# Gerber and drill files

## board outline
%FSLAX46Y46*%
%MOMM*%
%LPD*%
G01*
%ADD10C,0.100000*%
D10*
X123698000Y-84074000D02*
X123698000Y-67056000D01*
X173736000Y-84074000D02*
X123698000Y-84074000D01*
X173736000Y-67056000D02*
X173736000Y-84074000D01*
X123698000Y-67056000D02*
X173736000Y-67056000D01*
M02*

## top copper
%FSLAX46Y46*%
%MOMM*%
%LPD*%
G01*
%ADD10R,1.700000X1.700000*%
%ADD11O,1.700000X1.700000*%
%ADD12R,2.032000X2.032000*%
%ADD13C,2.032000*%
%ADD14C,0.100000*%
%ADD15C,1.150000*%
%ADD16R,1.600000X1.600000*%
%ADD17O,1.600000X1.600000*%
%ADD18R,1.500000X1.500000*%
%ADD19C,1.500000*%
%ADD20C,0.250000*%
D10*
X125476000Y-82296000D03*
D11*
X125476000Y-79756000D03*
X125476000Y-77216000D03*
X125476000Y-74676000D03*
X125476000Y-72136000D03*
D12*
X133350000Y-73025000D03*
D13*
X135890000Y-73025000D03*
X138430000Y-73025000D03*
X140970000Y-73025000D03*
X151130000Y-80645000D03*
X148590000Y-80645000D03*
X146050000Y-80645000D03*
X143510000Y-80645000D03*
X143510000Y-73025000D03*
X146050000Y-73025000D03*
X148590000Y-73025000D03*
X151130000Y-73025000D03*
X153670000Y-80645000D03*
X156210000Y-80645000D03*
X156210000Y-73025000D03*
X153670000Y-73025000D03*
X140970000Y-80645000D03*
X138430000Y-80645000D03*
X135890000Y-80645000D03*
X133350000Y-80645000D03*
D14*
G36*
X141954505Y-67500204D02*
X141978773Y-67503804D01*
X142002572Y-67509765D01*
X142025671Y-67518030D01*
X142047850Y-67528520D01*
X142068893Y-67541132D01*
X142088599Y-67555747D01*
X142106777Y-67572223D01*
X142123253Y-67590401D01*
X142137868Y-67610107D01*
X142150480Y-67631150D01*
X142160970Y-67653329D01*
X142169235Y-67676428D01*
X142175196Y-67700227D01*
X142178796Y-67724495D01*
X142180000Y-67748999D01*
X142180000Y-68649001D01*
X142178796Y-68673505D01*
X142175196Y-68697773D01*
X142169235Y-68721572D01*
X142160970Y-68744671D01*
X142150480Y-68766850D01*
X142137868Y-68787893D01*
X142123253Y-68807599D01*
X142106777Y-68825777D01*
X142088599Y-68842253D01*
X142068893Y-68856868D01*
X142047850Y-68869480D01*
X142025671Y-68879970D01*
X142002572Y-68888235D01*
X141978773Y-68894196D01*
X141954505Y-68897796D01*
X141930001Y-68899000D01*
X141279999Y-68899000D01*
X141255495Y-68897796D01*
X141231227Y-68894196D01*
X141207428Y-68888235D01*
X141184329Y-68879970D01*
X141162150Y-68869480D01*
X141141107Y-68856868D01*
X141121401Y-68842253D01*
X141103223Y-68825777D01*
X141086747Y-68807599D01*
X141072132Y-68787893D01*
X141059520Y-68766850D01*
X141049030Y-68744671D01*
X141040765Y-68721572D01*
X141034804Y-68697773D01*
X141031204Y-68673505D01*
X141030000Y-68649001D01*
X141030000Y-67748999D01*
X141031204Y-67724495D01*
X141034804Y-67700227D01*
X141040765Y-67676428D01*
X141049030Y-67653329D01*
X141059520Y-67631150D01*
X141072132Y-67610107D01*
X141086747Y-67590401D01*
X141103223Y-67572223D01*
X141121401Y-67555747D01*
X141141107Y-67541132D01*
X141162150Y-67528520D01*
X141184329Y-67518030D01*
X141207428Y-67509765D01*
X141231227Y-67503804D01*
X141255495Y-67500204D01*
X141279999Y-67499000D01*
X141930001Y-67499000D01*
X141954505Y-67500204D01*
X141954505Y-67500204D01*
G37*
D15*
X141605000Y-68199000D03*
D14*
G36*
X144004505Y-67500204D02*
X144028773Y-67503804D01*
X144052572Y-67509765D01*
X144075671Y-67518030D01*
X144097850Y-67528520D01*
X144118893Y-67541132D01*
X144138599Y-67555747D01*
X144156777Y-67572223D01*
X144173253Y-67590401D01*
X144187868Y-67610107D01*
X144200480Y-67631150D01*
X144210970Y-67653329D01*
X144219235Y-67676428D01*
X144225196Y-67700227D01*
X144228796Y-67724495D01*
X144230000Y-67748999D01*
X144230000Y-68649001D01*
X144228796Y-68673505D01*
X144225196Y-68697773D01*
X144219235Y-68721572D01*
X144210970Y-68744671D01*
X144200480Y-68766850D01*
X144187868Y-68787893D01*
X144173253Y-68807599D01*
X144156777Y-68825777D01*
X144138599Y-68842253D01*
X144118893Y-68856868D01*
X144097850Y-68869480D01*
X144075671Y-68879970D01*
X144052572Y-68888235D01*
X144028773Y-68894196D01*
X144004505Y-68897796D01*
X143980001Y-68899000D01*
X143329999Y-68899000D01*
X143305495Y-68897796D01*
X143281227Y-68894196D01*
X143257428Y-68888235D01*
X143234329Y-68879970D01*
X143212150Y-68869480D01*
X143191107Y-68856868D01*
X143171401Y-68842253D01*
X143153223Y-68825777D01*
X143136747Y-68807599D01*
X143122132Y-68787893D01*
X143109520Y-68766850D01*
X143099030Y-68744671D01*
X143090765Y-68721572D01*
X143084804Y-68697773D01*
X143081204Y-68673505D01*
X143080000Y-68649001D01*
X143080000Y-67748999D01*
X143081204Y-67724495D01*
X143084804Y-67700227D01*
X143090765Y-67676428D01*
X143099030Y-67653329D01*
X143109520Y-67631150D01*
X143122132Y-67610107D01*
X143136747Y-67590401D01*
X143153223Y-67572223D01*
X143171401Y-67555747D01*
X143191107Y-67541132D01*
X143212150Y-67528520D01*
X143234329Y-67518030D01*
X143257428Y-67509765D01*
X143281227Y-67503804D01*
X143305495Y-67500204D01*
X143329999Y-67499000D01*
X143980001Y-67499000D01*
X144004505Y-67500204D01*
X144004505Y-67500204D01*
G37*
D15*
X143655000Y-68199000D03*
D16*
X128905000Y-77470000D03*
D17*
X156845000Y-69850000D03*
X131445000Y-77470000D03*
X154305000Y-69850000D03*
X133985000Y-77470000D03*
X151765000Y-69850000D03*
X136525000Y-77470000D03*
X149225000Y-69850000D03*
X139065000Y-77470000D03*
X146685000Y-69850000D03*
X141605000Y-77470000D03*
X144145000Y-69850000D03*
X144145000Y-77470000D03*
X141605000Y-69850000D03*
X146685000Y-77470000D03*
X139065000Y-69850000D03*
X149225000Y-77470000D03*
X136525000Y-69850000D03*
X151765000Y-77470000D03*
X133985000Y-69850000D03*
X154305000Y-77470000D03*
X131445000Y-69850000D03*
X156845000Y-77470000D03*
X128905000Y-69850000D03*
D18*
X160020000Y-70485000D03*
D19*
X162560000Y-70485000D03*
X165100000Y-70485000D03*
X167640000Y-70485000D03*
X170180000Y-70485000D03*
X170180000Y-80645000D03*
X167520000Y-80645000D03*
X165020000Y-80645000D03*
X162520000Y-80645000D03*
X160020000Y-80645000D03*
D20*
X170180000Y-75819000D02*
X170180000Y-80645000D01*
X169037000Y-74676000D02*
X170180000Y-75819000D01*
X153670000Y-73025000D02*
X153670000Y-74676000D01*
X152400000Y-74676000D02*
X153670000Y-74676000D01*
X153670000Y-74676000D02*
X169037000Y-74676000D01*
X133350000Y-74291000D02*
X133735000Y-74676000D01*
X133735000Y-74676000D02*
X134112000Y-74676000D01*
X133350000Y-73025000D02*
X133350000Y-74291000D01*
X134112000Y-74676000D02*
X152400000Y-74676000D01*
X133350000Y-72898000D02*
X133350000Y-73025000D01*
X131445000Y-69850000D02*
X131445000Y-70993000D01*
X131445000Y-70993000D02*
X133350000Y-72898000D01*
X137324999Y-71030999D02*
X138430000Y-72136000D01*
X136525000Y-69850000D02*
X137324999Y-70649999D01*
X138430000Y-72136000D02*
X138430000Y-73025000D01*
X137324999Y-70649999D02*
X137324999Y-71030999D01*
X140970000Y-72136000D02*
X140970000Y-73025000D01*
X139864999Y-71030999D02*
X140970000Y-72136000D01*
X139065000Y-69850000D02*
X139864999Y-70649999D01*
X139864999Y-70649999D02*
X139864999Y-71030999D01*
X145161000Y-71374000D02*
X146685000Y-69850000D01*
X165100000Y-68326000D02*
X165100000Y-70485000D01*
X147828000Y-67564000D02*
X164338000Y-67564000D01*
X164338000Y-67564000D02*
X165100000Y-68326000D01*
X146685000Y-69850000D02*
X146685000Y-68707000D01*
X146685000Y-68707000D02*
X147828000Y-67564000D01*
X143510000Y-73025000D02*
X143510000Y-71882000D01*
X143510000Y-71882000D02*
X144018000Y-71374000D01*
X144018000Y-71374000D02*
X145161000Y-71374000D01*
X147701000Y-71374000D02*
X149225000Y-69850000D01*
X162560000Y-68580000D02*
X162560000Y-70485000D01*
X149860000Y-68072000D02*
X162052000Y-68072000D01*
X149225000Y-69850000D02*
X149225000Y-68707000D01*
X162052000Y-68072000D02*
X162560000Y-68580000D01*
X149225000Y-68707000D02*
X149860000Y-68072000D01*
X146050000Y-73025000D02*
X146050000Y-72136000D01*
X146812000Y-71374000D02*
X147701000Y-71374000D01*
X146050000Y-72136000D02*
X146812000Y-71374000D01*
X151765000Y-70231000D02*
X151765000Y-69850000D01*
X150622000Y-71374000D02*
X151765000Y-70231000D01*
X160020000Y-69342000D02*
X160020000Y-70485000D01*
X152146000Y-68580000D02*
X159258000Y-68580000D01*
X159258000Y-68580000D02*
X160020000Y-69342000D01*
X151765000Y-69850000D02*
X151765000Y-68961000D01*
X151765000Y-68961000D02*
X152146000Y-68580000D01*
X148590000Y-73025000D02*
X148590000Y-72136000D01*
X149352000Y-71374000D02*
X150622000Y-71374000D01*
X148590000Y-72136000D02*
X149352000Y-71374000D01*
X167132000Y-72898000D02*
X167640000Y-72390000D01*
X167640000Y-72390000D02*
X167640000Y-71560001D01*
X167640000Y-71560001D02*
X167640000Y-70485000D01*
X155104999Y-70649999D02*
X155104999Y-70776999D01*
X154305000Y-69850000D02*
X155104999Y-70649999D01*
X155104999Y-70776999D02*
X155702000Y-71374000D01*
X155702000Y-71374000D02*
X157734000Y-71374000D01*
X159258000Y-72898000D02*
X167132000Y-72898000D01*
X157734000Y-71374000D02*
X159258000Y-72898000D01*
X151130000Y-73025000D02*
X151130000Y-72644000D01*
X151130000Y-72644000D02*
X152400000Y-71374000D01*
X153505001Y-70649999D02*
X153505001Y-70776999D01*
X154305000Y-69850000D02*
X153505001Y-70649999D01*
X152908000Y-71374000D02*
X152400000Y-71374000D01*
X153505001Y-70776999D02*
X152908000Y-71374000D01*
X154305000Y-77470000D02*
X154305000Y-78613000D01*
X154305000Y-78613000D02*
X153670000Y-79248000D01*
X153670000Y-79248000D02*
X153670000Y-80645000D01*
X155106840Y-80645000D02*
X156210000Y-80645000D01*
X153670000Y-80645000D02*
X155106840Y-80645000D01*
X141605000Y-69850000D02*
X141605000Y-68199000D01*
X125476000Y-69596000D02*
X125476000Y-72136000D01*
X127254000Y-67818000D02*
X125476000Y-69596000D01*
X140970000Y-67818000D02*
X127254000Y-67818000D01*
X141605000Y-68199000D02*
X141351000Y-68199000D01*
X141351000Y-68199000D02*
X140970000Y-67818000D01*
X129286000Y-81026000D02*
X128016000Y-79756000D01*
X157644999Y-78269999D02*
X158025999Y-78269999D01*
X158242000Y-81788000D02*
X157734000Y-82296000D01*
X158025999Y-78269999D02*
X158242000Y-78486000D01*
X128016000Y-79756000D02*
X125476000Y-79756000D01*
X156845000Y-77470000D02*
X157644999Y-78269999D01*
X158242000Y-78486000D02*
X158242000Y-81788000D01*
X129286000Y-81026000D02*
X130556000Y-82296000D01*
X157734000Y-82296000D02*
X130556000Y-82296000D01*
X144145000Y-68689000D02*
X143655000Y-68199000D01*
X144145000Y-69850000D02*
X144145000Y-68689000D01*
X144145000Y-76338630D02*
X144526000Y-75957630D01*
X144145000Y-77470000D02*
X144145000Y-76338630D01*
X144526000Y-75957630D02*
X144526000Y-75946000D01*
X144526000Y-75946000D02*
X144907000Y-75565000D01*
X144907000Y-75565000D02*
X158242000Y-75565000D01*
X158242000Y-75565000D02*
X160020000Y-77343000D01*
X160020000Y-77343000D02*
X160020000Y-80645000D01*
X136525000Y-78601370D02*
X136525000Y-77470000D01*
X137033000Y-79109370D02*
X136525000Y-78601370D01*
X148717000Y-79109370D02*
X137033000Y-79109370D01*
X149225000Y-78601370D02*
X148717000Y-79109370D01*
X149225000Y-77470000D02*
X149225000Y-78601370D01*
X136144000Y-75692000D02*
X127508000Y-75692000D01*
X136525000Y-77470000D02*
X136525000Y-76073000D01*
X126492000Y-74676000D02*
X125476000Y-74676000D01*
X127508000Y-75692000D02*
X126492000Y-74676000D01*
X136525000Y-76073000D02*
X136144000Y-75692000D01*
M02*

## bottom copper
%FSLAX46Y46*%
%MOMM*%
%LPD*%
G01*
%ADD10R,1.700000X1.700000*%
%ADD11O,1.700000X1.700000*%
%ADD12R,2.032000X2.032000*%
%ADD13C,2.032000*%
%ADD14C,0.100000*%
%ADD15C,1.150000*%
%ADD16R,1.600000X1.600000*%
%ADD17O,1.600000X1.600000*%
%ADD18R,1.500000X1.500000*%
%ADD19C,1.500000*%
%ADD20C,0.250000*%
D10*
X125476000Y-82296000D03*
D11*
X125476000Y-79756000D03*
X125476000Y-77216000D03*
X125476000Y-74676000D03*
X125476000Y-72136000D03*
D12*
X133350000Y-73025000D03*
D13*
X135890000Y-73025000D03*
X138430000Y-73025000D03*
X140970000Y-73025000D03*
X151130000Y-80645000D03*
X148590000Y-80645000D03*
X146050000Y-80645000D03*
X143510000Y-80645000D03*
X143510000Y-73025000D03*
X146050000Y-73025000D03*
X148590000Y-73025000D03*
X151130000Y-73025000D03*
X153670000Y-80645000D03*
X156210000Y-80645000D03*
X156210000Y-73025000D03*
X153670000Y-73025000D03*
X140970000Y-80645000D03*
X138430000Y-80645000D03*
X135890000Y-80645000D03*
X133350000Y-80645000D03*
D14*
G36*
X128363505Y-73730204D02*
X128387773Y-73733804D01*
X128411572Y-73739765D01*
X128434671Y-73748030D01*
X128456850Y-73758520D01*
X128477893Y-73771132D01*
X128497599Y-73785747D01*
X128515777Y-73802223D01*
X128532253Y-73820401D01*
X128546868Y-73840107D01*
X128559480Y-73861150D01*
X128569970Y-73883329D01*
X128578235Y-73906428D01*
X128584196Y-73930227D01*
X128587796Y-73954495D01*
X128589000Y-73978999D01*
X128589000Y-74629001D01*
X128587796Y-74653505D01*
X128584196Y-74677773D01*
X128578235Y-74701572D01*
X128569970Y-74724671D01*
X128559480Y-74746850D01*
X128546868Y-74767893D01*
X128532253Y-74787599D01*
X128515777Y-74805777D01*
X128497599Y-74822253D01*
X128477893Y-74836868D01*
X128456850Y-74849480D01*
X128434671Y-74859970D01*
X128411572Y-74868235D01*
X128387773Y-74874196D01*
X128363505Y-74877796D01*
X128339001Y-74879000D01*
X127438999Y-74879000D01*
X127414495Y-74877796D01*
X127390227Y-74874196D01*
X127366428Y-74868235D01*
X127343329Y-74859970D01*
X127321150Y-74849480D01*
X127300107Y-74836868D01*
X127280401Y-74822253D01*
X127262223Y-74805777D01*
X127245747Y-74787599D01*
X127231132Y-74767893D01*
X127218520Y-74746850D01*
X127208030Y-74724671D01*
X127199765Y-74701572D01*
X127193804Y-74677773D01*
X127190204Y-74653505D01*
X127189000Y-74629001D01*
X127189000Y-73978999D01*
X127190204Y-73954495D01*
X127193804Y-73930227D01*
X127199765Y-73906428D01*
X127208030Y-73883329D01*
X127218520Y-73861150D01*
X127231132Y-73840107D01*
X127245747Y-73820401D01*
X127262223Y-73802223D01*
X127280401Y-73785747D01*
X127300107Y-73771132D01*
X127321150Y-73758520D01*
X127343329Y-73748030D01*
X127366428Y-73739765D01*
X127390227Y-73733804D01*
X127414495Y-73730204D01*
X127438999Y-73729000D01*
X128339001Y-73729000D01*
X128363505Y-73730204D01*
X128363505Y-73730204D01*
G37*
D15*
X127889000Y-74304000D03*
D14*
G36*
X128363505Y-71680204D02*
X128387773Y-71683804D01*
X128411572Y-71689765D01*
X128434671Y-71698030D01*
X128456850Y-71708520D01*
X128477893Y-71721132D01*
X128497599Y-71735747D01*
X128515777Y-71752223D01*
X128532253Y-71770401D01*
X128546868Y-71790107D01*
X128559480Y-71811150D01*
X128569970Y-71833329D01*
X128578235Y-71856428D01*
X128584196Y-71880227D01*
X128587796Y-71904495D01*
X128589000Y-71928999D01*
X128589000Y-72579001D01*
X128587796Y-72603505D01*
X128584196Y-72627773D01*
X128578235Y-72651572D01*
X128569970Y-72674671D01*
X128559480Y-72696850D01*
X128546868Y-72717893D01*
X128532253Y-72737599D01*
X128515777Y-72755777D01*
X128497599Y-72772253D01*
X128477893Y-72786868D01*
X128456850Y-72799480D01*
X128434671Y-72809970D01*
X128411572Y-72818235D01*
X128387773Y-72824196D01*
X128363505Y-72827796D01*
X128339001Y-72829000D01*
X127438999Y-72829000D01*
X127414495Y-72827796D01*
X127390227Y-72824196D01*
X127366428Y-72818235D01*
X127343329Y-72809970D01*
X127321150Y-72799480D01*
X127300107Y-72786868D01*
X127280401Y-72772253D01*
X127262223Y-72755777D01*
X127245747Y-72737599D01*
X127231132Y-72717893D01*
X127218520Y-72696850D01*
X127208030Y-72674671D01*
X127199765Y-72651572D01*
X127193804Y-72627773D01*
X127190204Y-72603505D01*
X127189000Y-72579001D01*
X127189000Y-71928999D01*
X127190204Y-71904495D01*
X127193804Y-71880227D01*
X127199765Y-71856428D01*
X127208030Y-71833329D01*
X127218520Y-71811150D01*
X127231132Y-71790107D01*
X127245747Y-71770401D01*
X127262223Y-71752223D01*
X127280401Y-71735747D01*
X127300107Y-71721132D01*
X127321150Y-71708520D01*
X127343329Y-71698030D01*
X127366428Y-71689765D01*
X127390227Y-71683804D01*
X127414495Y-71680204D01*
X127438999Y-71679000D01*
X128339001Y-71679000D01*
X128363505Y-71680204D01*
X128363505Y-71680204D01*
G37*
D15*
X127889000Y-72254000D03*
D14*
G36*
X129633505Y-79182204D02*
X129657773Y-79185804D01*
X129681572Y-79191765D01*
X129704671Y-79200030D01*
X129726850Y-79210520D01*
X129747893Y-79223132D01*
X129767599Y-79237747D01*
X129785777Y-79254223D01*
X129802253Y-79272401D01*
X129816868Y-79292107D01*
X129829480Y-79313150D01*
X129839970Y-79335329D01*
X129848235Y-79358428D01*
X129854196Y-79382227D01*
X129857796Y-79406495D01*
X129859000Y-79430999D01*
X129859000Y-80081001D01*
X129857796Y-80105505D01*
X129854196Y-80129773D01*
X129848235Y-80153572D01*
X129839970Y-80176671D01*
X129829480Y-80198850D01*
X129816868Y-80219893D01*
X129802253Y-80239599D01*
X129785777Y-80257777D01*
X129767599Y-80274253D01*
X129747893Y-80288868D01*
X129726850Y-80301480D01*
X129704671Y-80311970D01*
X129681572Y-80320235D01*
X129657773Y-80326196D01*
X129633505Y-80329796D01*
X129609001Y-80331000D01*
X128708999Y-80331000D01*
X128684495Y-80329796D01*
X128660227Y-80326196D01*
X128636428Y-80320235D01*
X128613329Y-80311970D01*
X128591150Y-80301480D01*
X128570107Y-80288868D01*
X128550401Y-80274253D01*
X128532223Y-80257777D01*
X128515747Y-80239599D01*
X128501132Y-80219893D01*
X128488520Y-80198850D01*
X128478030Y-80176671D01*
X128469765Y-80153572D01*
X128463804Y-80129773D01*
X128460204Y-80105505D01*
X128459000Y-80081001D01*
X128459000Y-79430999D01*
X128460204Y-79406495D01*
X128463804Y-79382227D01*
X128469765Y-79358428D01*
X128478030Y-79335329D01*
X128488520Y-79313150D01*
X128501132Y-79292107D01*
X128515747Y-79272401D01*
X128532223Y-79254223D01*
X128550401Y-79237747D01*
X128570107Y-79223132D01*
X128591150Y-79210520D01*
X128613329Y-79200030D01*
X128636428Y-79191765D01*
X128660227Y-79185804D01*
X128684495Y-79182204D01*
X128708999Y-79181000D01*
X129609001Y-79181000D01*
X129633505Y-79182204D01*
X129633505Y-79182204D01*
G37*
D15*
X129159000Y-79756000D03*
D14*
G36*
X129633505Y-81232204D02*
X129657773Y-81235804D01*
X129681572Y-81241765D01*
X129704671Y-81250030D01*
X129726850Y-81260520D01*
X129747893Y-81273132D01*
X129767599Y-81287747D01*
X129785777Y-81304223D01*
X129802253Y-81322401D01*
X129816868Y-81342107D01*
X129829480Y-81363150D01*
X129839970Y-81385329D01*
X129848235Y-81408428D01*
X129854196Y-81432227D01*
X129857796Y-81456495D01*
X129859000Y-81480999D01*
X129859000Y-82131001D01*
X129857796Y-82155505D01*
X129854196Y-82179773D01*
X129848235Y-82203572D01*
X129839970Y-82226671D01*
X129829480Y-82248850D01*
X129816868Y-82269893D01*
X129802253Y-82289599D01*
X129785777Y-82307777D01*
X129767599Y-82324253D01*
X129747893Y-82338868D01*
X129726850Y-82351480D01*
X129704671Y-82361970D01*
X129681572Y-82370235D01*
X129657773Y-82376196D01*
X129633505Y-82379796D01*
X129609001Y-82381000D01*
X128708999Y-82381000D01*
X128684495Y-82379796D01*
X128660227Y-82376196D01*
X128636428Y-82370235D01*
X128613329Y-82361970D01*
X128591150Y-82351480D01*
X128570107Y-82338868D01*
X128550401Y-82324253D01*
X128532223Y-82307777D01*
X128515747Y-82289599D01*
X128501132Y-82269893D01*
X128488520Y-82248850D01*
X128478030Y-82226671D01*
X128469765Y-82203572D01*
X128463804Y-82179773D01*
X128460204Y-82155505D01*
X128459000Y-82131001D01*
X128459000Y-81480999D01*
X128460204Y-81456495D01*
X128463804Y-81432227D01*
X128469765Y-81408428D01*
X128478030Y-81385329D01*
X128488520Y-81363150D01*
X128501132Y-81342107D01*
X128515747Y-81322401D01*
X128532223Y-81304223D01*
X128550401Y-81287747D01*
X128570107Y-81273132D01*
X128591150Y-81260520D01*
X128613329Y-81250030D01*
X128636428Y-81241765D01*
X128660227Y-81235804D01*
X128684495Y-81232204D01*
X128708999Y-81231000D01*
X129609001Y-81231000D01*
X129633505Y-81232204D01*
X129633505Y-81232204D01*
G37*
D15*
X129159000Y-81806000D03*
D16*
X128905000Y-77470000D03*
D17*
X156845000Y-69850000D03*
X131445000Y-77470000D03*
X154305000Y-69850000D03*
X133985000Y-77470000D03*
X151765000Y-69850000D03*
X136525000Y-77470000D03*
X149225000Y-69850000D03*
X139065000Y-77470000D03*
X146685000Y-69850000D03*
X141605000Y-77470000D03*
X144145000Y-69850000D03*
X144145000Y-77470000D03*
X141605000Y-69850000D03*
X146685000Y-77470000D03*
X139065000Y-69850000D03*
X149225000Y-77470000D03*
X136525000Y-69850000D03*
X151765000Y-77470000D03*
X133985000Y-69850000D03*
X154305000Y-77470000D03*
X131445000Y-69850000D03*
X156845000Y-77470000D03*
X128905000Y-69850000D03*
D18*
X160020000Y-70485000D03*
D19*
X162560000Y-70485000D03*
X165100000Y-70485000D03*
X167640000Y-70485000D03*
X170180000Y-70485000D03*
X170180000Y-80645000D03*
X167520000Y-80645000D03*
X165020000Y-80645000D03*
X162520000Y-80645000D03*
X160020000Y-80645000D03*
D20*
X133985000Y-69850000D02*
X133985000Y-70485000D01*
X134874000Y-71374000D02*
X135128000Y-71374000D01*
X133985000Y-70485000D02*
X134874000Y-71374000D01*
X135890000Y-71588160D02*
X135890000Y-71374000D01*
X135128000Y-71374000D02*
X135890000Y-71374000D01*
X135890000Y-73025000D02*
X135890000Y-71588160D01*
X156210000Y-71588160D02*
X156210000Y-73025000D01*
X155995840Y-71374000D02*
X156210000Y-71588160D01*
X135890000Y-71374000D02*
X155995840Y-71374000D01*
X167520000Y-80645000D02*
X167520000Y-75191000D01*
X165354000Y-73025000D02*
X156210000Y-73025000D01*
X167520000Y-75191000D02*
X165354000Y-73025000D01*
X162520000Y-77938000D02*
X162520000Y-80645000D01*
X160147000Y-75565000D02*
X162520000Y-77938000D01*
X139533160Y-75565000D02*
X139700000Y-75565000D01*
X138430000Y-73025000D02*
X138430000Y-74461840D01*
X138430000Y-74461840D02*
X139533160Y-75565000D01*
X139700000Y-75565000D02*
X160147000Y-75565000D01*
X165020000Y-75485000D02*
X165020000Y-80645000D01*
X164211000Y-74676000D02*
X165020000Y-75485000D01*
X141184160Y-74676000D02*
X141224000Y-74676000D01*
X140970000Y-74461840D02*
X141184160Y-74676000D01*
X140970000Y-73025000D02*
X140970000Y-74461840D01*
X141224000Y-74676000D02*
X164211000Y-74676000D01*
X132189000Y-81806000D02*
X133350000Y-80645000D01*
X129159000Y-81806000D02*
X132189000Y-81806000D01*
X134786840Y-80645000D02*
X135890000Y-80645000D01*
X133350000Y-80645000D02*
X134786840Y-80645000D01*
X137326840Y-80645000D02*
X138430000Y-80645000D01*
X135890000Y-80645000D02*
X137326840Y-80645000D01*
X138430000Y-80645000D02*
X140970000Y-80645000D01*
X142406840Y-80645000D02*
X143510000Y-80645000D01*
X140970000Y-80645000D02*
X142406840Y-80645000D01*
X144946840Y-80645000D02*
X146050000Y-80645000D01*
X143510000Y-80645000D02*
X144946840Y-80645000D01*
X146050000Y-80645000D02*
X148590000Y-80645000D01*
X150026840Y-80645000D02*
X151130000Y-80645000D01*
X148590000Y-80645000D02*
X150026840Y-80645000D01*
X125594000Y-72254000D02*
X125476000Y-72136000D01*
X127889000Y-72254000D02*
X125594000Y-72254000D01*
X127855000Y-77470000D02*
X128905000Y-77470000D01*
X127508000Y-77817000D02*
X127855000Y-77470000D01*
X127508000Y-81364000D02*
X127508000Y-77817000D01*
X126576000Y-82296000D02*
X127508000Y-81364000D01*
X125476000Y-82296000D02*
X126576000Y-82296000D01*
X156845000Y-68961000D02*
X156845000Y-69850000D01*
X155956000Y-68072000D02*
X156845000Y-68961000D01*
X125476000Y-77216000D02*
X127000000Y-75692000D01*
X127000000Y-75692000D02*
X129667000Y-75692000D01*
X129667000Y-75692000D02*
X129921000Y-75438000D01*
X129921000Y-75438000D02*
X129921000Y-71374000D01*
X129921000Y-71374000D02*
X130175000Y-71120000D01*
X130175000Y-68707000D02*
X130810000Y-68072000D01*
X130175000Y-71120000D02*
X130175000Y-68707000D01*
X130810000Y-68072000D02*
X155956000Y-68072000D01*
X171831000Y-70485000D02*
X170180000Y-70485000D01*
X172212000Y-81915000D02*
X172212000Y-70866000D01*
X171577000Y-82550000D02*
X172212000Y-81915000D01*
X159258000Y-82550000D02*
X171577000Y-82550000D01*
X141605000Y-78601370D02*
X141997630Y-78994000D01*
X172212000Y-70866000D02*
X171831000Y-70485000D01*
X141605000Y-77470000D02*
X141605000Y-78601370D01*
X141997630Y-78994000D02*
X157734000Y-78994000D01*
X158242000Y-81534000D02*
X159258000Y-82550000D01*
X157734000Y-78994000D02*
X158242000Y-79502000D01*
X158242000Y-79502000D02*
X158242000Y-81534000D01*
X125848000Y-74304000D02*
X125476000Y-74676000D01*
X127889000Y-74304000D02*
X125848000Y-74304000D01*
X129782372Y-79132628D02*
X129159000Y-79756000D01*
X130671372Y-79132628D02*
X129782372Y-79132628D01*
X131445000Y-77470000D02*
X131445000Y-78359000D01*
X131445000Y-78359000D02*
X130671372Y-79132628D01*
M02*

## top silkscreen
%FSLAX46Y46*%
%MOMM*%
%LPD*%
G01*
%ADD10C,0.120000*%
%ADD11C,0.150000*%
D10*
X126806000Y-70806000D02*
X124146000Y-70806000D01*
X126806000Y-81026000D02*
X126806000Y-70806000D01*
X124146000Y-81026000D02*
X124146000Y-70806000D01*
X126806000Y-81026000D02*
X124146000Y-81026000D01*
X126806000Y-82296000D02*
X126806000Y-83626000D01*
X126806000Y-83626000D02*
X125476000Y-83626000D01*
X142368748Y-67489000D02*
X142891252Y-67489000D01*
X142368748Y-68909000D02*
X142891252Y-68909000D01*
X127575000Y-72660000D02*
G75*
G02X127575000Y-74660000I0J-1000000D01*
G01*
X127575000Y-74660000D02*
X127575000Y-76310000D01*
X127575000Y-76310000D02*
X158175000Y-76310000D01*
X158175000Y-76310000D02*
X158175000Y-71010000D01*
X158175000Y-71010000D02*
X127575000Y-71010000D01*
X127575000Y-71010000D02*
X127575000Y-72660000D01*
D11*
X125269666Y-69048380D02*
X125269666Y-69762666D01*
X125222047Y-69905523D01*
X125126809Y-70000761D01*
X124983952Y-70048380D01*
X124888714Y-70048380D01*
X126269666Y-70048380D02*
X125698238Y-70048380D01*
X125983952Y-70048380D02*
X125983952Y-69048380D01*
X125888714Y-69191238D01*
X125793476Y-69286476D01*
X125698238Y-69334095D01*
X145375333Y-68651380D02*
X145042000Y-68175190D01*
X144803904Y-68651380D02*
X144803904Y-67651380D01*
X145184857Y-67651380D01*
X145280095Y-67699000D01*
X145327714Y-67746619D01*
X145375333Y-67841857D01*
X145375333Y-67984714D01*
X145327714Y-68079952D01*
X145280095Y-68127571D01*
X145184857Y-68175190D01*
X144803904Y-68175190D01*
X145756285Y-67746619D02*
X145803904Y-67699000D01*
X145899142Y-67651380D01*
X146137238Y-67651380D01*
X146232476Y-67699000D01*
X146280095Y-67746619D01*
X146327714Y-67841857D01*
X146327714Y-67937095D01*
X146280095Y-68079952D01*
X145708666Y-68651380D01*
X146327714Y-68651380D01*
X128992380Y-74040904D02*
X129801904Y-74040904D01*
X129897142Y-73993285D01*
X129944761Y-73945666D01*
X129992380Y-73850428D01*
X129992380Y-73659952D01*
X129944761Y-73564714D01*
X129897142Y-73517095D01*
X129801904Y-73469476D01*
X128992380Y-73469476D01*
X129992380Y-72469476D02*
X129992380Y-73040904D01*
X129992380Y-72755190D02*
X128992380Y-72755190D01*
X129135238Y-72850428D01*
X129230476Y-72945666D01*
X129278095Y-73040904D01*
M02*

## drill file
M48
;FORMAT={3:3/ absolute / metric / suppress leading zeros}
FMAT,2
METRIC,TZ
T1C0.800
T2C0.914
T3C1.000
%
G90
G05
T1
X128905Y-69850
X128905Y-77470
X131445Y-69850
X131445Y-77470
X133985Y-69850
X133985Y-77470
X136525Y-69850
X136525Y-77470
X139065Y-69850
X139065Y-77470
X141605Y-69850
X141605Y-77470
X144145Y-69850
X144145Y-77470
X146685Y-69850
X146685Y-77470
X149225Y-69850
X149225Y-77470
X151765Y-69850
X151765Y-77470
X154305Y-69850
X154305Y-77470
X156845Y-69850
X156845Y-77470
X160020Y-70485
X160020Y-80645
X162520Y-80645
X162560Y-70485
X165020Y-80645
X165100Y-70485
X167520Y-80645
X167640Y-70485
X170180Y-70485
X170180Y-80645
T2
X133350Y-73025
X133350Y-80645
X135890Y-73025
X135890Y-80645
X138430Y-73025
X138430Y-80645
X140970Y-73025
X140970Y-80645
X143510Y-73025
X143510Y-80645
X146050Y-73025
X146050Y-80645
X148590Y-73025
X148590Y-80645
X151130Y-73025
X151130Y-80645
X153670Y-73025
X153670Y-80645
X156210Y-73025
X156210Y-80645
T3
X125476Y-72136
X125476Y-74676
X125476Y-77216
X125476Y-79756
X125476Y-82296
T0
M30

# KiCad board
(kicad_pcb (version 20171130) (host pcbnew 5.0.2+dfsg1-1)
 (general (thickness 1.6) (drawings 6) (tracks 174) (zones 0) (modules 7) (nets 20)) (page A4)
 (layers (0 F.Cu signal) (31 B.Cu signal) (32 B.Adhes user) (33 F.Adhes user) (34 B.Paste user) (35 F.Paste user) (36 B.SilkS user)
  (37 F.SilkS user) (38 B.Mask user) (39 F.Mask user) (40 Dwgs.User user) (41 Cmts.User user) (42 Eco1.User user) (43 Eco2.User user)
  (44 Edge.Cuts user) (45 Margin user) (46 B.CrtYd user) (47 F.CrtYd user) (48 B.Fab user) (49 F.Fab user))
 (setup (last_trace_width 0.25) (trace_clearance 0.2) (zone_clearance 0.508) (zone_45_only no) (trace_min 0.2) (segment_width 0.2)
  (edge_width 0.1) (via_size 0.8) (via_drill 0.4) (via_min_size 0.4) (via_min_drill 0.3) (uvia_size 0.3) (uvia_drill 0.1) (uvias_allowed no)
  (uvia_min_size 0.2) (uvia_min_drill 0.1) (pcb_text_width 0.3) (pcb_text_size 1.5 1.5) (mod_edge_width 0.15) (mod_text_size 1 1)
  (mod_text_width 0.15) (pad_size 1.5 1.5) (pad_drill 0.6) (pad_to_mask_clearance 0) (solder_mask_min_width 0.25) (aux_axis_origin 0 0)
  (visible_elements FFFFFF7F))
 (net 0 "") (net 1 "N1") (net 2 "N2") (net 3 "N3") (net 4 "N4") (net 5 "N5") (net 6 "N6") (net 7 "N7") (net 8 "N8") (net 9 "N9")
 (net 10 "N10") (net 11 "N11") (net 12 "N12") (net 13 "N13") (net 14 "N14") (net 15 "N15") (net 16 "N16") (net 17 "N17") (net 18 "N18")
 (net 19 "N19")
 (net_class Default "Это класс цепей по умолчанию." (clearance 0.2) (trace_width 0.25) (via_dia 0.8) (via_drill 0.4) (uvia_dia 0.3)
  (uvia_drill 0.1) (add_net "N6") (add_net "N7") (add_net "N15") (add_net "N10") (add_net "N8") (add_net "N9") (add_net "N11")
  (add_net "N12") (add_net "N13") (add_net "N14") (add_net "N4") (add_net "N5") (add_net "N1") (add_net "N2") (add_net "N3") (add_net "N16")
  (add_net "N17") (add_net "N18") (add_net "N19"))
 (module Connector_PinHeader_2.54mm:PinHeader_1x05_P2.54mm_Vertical (layer F.Cu) (at 125.476 82.296 180)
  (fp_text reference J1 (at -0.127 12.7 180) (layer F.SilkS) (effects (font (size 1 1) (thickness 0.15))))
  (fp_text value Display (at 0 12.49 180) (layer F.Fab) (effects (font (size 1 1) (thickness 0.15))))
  (fp_line (start -1.33 11.49) (end 1.33 11.49) (layer F.SilkS) (width 0.12))
  (fp_line (start -1.33 1.27) (end -1.33 11.49) (layer F.SilkS) (width 0.12))
  (fp_line (start 1.33 1.27) (end 1.33 11.49) (layer F.SilkS) (width 0.12))
  (fp_line (start -1.33 1.27) (end 1.33 1.27) (layer F.SilkS) (width 0.12))
  (fp_line (start -1.33 0) (end -1.33 -1.33) (layer F.SilkS) (width 0.12))
  (fp_line (start -1.33 -1.33) (end 0 -1.33) (layer F.SilkS) (width 0.12))
  (pad 1 thru_hole rect (at 0 0 180) (size 1.7 1.7) (drill 1) (layers *.Cu *.Mask) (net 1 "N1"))
  (pad 2 thru_hole oval (at 0 2.54 180) (size 1.7 1.7) (drill 1) (layers *.Cu *.Mask) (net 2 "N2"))
  (pad 3 thru_hole oval (at 0 5.08 180) (size 1.7 1.7) (drill 1) (layers *.Cu *.Mask) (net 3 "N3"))
  (pad 4 thru_hole oval (at 0 7.62 180) (size 1.7 1.7) (drill 1) (layers *.Cu *.Mask) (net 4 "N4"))
  (pad 5 thru_hole oval (at 0 10.16 180) (size 1.7 1.7) (drill 1) (layers *.Cu *.Mask) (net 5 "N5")))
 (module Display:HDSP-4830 (layer B.Cu) (at 133.35 73.025 270)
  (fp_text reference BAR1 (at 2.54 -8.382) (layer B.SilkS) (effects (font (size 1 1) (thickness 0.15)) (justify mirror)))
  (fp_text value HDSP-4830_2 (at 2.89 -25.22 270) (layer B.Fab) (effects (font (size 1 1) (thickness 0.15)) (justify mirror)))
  (pad 1 thru_hole rect (at 0 0) (size 2.032 2.032) (drill 0.9144) (layers *.Cu *.Mask) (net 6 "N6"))
  (pad 2 thru_hole circle (at 0 -2.54) (size 2.032 2.032) (drill 0.9144) (layers *.Cu *.Mask) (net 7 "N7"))
  (pad 3 thru_hole circle (at 0 -5.08) (size 2.032 2.032) (drill 0.9144) (layers *.Cu *.Mask) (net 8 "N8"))
  (pad 4 thru_hole circle (at 0 -7.62) (size 2.032 2.032) (drill 0.9144) (layers *.Cu *.Mask) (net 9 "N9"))
  (pad 13 thru_hole circle (at 7.62 -17.78) (size 2.032 2.032) (drill 0.9144) (layers *.Cu *.Mask) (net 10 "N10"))
  (pad 14 thru_hole circle (at 7.62 -15.24) (size 2.032 2.032) (drill 0.9144) (layers *.Cu *.Mask) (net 10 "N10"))
  (pad 15 thru_hole circle (at 7.62 -12.7) (size 2.032 2.032) (drill 0.9144) (layers *.Cu *.Mask) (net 10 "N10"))
  (pad 16 thru_hole circle (at 7.62 -10.16) (size 2.032 2.032) (drill 0.9144) (layers *.Cu *.Mask) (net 10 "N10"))
  (pad 5 thru_hole circle (at 0 -10.16) (size 2.032 2.032) (drill 0.9144) (layers *.Cu *.Mask) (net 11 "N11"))
  (pad 6 thru_hole circle (at 0 -12.7) (size 2.032 2.032) (drill 0.9144) (layers *.Cu *.Mask) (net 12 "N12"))
  (pad 7 thru_hole circle (at 0 -15.24) (size 2.032 2.032) (drill 0.9144) (layers *.Cu *.Mask) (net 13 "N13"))
  (pad 8 thru_hole circle (at 0 -17.78) (size 2.032 2.032) (drill 0.9144) (layers *.Cu *.Mask) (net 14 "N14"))
  (pad 12 thru_hole circle (at 7.62 -20.32) (size 2.032 2.032) (drill 0.9144) (layers *.Cu *.Mask) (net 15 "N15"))
  (pad 11 thru_hole circle (at 7.62 -22.86) (size 2.032 2.032) (drill 0.9144) (layers *.Cu *.Mask) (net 15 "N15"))
  (pad 10 thru_hole circle (at 0 -22.86) (size 2.032 2.032) (drill 0.9144) (layers *.Cu *.Mask) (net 7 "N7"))
  (pad 9 thru_hole circle (at 0 -20.32) (size 2.032 2.032) (drill 0.9144) (layers *.Cu *.Mask) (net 6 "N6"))
  (pad 17 thru_hole circle (at 7.62 -7.62) (size 2.032 2.032) (drill 0.9144) (layers *.Cu *.Mask) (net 10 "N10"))
  (pad 18 thru_hole circle (at 7.62 -5.08) (size 2.032 2.032) (drill 0.9144) (layers *.Cu *.Mask) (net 10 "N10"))
  (pad 19 thru_hole circle (at 7.62 -2.54) (size 2.032 2.032) (drill 0.9144) (layers *.Cu *.Mask) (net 10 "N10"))
  (pad 20 thru_hole circle (at 7.62 0) (size 2.032 2.032) (drill 0.9144) (layers *.Cu *.Mask) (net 10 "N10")))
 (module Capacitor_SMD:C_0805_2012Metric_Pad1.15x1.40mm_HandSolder (layer B.Cu) (at 127.889 73.279 90)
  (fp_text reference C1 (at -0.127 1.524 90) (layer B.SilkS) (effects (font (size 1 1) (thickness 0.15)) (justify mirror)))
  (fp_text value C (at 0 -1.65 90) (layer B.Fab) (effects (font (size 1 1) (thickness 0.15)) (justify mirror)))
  (pad 1 smd roundrect (at -1.025 0 90) (size 1.15 1.4) (layers B.Cu B.Paste B.Mask) (roundrect_rratio 0.217391) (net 4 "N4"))
  (pad 2 smd roundrect (at 1.025 0 90) (size 1.15 1.4) (layers B.Cu B.Paste B.Mask) (roundrect_rratio 0.217391) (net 5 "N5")))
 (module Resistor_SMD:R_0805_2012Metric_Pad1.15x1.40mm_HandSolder (layer B.Cu) (at 129.159 80.781 90)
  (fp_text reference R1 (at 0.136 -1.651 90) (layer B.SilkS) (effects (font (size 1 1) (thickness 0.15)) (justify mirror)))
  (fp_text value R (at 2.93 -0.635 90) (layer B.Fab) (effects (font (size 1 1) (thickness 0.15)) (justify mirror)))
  (pad 2 smd roundrect (at 1.025 0 90) (size 1.15 1.4) (layers B.Cu B.Paste B.Mask) (roundrect_rratio 0.217391) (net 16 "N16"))
  (pad 1 smd roundrect (at -1.025 0 90) (size 1.15 1.4) (layers B.Cu B.Paste B.Mask) (roundrect_rratio 0.217391) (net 10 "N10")))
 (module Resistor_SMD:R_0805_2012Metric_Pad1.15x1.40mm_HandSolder (layer F.Cu) (at 142.63 68.199)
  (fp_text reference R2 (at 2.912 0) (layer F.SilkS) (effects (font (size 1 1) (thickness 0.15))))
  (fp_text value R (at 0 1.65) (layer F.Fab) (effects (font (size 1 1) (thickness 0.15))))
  (fp_line (start -0.261252 -0.71) (end 0.261252 -0.71) (layer F.SilkS) (width 0.12))
  (fp_line (start -0.261252 0.71) (end 0.261252 0.71) (layer F.SilkS) (width 0.12))
  (pad 1 smd roundrect (at -1.025 0) (size 1.15 1.4) (layers F.Cu F.Paste F.Mask) (roundrect_rratio 0.217391) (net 5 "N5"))
  (pad 2 smd roundrect (at 1.025 0) (size 1.15 1.4) (layers F.Cu F.Paste F.Mask) (roundrect_rratio 0.217391) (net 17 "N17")))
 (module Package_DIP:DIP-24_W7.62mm (layer F.Cu) (at 128.905 77.47 90)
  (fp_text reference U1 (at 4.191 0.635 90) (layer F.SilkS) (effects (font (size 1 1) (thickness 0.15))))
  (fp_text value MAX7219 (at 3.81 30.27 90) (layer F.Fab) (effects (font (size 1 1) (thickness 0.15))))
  (fp_arc (start 3.81 -1.33) (end 2.81 -1.33) (angle -180) (layer F.SilkS) (width 0.12))
  (fp_line (start 2.81 -1.33) (end 1.16 -1.33) (layer F.SilkS) (width 0.12))
  (fp_line (start 1.16 -1.33) (end 1.16 29.27) (layer F.SilkS) (width 0.12))
  (fp_line (start 1.16 29.27) (end 6.46 29.27) (layer F.SilkS) (width 0.12))
  (fp_line (start 6.46 29.27) (end 6.46 -1.33) (layer F.SilkS) (width 0.12))
  (fp_line (start 6.46 -1.33) (end 4.81 -1.33) (layer F.SilkS) (width 0.12))
  (pad 1 thru_hole rect (at 0 0 90) (size 1.6 1.6) (drill 0.8) (layers *.Cu *.Mask) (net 1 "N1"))
  (pad 13 thru_hole oval (at 7.62 27.94 90) (size 1.6 1.6) (drill 0.8) (layers *.Cu *.Mask) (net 3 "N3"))
  (pad 2 thru_hole oval (at 0 2.54 90) (size 1.6 1.6) (drill 0.8) (layers *.Cu *.Mask) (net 16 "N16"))
  (pad 14 thru_hole oval (at 7.62 25.4 90) (size 1.6 1.6) (drill 0.8) (layers *.Cu *.Mask) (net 14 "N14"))
  (pad 3 thru_hole oval (at 0 5.08 90) (size 1.6 1.6) (drill 0.8) (layers *.Cu *.Mask))
  (pad 15 thru_hole oval (at 7.62 22.86 90) (size 1.6 1.6) (drill 0.8) (layers *.Cu *.Mask) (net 13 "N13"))
  (pad 4 thru_hole oval (at 0 7.62 90) (size 1.6 1.6) (drill 0.8) (layers *.Cu *.Mask) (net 4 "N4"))
  (pad 16 thru_hole oval (at 7.62 20.32 90) (size 1.6 1.6) (drill 0.8) (layers *.Cu *.Mask) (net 12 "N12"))
  (pad 5 thru_hole oval (at 0 10.16 90) (size 1.6 1.6) (drill 0.8) (layers *.Cu *.Mask))
  (pad 17 thru_hole oval (at 7.62 17.78 90) (size 1.6 1.6) (drill 0.8) (layers *.Cu *.Mask) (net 11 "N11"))
  (pad 6 thru_hole oval (at 0 12.7 90) (size 1.6 1.6) (drill 0.8) (layers *.Cu *.Mask) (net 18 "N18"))
  (pad 18 thru_hole oval (at 7.62 15.24 90) (size 1.6 1.6) (drill 0.8) (layers *.Cu *.Mask) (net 17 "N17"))
  (pad 7 thru_hole oval (at 0 15.24 90) (size 1.6 1.6) (drill 0.8) (layers *.Cu *.Mask) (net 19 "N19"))
  (pad 19 thru_hole oval (at 7.62 12.7 90) (size 1.6 1.6) (drill 0.8) (layers *.Cu *.Mask) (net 5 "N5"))
  (pad 8 thru_hole oval (at 0 17.78 90) (size 1.6 1.6) (drill 0.8) (layers *.Cu *.Mask))
  (pad 20 thru_hole oval (at 7.62 10.16 90) (size 1.6 1.6) (drill 0.8) (layers *.Cu *.Mask) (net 9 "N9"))
  (pad 9 thru_hole oval (at 0 20.32 90) (size 1.6 1.6) (drill 0.8) (layers *.Cu *.Mask) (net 4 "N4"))
  (pad 21 thru_hole oval (at 7.62 7.62 90) (size 1.6 1.6) (drill 0.8) (layers *.Cu *.Mask) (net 8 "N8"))
  (pad 10 thru_hole oval (at 0 22.86 90) (size 1.6 1.6) (drill 0.8) (layers *.Cu *.Mask))
  (pad 22 thru_hole oval (at 7.62 5.08 90) (size 1.6 1.6) (drill 0.8) (layers *.Cu *.Mask) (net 7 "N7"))
  (pad 11 thru_hole oval (at 0 25.4 90) (size 1.6 1.6) (drill 0.8) (layers *.Cu *.Mask) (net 15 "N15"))
  (pad 23 thru_hole oval (at 7.62 2.54 90) (size 1.6 1.6) (drill 0.8) (layers *.Cu *.Mask) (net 6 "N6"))
  (pad 12 thru_hole oval (at 0 27.94 90) (size 1.6 1.6) (drill 0.8) (layers *.Cu *.Mask) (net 2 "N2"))
  (pad 24 thru_hole oval (at 7.62 0 90) (size 1.6 1.6) (drill 0.8) (layers *.Cu *.Mask)))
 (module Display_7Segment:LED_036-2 (layer B.Cu) (at 160.02 70.485 270)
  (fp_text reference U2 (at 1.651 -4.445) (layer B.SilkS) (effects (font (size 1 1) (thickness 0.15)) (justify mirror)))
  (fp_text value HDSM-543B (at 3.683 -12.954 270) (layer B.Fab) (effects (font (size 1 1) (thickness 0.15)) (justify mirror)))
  (pad 1 thru_hole rect (at 0 0 270) (size 1.5 1.5) (drill 0.8) (layers *.Cu *.Mask) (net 13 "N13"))
  (pad 2 thru_hole circle (at 0 -2.54 270) (size 1.5 1.5) (drill 0.8) (layers *.Cu *.Mask) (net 12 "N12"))
  (pad 3 thru_hole circle (at 0 -5.08 270) (size 1.5 1.5) (drill 0.8) (layers *.Cu *.Mask) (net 11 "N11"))
  (pad 4 thru_hole circle (at 0 -7.62 270) (size 1.5 1.5) (drill 0.8) (layers *.Cu *.Mask) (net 14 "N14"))
  (pad 5 thru_hole circle (at 0 -10.16 270) (size 1.5 1.5) (drill 0.8) (layers *.Cu *.Mask) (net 18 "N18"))
  (pad 6 thru_hole circle (at 10.16 -10.16 270) (size 1.5 1.5) (drill 0.8) (layers *.Cu *.Mask) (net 6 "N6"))
  (pad 7 thru_hole circle (at 10.16 -7.5 270) (size 1.5 1.5) (drill 0.8) (layers *.Cu *.Mask) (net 7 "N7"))
  (pad 8 thru_hole circle (at 10.16 -5 270) (size 1.5 1.5) (drill 0.8) (layers *.Cu *.Mask) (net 9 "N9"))
  (pad 9 thru_hole circle (at 10.16 -2.5 270) (size 1.5 1.5) (drill 0.8) (layers *.Cu *.Mask) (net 8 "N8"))
  (pad 10 thru_hole circle (at 10.16 0 270) (size 1.5 1.5) (drill 0.8) (layers *.Cu *.Mask) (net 19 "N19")))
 (gr_line (start 123.698 84.074) (end 123.698 67.056) (layer Edge.Cuts) (width 0.1))
 (gr_line (start 173.736 84.074) (end 123.698 84.074) (layer Edge.Cuts) (width 0.1))
 (gr_line (start 173.736 67.056) (end 173.736 84.074) (layer Edge.Cuts) (width 0.1))
 (gr_line (start 123.698 67.056) (end 173.736 67.056) (layer Edge.Cuts) (width 0.1))
 (segment (start 170.18 75.819) (end 170.18 80.645) (width 0.25) (layer F.Cu) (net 6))
 (segment (start 169.037 74.676) (end 170.18 75.819) (width 0.25) (layer F.Cu) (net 6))
 (segment (start 153.67 73.025) (end 153.67 74.676) (width 0.25) (layer F.Cu) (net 6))
 (segment (start 152.4 74.676) (end 153.67 74.676) (width 0.25) (layer F.Cu) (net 6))
 (segment (start 153.67 74.676) (end 169.037 74.676) (width 0.25) (layer F.Cu) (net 6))
 (segment (start 133.35 74.291) (end 133.735 74.676) (width 0.25) (layer F.Cu) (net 6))
 (segment (start 133.735 74.676) (end 134.112 74.676) (width 0.25) (layer F.Cu) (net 6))
 (segment (start 133.35 73.025) (end 133.35 74.291) (width 0.25) (layer F.Cu) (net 6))
 (segment (start 134.112 74.676) (end 152.4 74.676) (width 0.25) (layer F.Cu) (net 6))
 (segment (start 133.35 72.898) (end 133.35 73.025) (width 0.25) (layer F.Cu) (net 6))
 (segment (start 131.445 69.85) (end 131.445 70.993) (width 0.25) (layer F.Cu) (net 6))
 (segment (start 131.445 70.993) (end 133.35 72.898) (width 0.25) (layer F.Cu) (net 6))
 (segment (start 133.985 69.85) (end 133.985 70.485) (width 0.25) (layer B.Cu) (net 7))
 (segment (start 134.874 71.374) (end 135.128 71.374) (width 0.25) (layer B.Cu) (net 7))
 (segment (start 133.985 70.485) (end 134.874 71.374) (width 0.25) (layer B.Cu) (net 7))
 (segment (start 135.89 71.58816) (end 135.89 71.374) (width 0.25) (layer B.Cu) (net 7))
 (segment (start 135.128 71.374) (end 135.89 71.374) (width 0.25) (layer B.Cu) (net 7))
 (segment (start 135.89 73.025) (end 135.89 71.58816) (width 0.25) (layer B.Cu) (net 7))
 (segment (start 156.21 71.58816) (end 156.21 73.025) (width 0.25) (layer B.Cu) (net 7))
 (segment (start 155.99584 71.374) (end 156.21 71.58816) (width 0.25) (layer B.Cu) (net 7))
 (segment (start 135.89 71.374) (end 155.99584 71.374) (width 0.25) (layer B.Cu) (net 7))
 (segment (start 167.52 80.645) (end 167.52 75.191) (width 0.25) (layer B.Cu) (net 7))
 (segment (start 165.354 73.025) (end 156.21 73.025) (width 0.25) (layer B.Cu) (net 7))
 (segment (start 167.52 75.191) (end 165.354 73.025) (width 0.25) (layer B.Cu) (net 7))
 (segment (start 162.52 77.938) (end 162.52 80.645) (width 0.25) (layer B.Cu) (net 8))
 (segment (start 160.147 75.565) (end 162.52 77.938) (width 0.25) (layer B.Cu) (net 8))
 (segment (start 139.53316 75.565) (end 139.7 75.565) (width 0.25) (layer B.Cu) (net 8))
 (segment (start 138.43 73.025) (end 138.43 74.46184) (width 0.25) (layer B.Cu) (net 8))
 (segment (start 138.43 74.46184) (end 139.53316 75.565) (width 0.25) (layer B.Cu) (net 8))
 (segment (start 139.7 75.565) (end 160.147 75.565) (width 0.25) (layer B.Cu) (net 8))
 (segment (start 137.324999 71.030999) (end 138.43 72.136) (width 0.25) (layer F.Cu) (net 8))
 (segment (start 136.525 69.85) (end 137.324999 70.649999) (width 0.25) (layer F.Cu) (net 8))
 (segment (start 138.43 72.136) (end 138.43 73.025) (width 0.25) (layer F.Cu) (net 8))
 (segment (start 137.324999 70.649999) (end 137.324999 71.030999) (width 0.25) (layer F.Cu) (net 8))
 (segment (start 165.02 75.485) (end 165.02 80.645) (width 0.25) (layer B.Cu) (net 9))
 (segment (start 164.211 74.676) (end 165.02 75.485) (width 0.25) (layer B.Cu) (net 9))
 (segment (start 141.18416 74.676) (end 141.224 74.676) (width 0.25) (layer B.Cu) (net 9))
 (segment (start 140.97 74.46184) (end 141.18416 74.676) (width 0.25) (layer B.Cu) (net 9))
 (segment (start 140.97 73.025) (end 140.97 74.46184) (width 0.25) (layer B.Cu) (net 9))
 (segment (start 141.224 74.676) (end 164.211 74.676) (width 0.25) (layer B.Cu) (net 9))
 (segment (start 140.97 72.136) (end 140.97 73.025) (width 0.25) (layer F.Cu) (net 9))
 (segment (start 139.864999 71.030999) (end 140.97 72.136) (width 0.25) (layer F.Cu) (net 9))
 (segment (start 139.065 69.85) (end 139.864999 70.649999) (width 0.25) (layer F.Cu) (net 9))
 (segment (start 139.864999 70.649999) (end 139.864999 71.030999) (width 0.25) (layer F.Cu) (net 9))
 (segment (start 132.189 81.806) (end 133.35 80.645) (width 0.25) (layer B.Cu) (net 10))
 (segment (start 129.159 81.806) (end 132.189 81.806) (width 0.25) (layer B.Cu) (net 10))
 (segment (start 134.78684 80.645) (end 135.89 80.645) (width 0.25) (layer B.Cu) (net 10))
 (segment (start 133.35 80.645) (end 134.78684 80.645) (width 0.25) (layer B.Cu) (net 10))
 (segment (start 137.32684 80.645) (end 138.43 80.645) (width 0.25) (layer B.Cu) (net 10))
 (segment (start 135.89 80.645) (end 137.32684 80.645) (width 0.25) (layer B.Cu) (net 10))
 (segment (start 138.43 80.645) (end 140.97 80.645) (width 0.25) (layer B.Cu) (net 10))
 (segment (start 142.40684 80.645) (end 143.51 80.645) (width 0.25) (layer B.Cu) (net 10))
 (segment (start 140.97 80.645) (end 142.40684 80.645) (width 0.25) (layer B.Cu) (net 10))
 (segment (start 144.94684 80.645) (end 146.05 80.645) (width 0.25) (layer B.Cu) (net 10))
 (segment (start 143.51 80.645) (end 144.94684 80.645) (width 0.25) (layer B.Cu) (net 10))
 (segment (start 146.05 80.645) (end 148.59 80.645) (width 0.25) (layer B.Cu) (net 10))
 (segment (start 150.02684 80.645) (end 151.13 80.645) (width 0.25) (layer B.Cu) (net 10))
 (segment (start 148.59 80.645) (end 150.02684 80.645) (width 0.25) (layer B.Cu) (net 10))
 (segment (start 145.161 71.374) (end 146.685 69.85) (width 0.25) (layer F.Cu) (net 11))
 (segment (start 165.1 68.326) (end 165.1 70.485) (width 0.25) (layer F.Cu) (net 11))
 (segment (start 147.828 67.564) (end 164.338 67.564) (width 0.25) (layer F.Cu) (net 11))
 (segment (start 164.338 67.564) (end 165.1 68.326) (width 0.25) (layer F.Cu) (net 11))
 (segment (start 146.685 69.85) (end 146.685 68.707) (width 0.25) (layer F.Cu) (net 11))
 (segment (start 146.685 68.707) (end 147.828 67.564) (width 0.25) (layer F.Cu) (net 11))
 (segment (start 143.51 73.025) (end 143.51 71.882) (width 0.25) (layer F.Cu) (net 11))
 (segment (start 143.51 71.882) (end 144.018 71.374) (width 0.25) (layer F.Cu) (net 11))
 (segment (start 144.018 71.374) (end 145.161 71.374) (width 0.25) (layer F.Cu) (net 11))
 (segment (start 147.701 71.374) (end 149.225 69.85) (width 0.25) (layer F.Cu) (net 12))
 (segment (start 162.56 68.58) (end 162.56 70.485) (width 0.25) (layer F.Cu) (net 12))
 (segment (start 149.86 68.072) (end 162.052 68.072) (width 0.25) (layer F.Cu) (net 12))
 (segment (start 149.225 69.85) (end 149.225 68.707) (width 0.25) (layer F.Cu) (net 12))
 (segment (start 162.052 68.072) (end 162.56 68.58) (width 0.25) (layer F.Cu) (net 12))
 (segment (start 149.225 68.707) (end 149.86 68.072) (width 0.25) (layer F.Cu) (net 12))
 (segment (start 146.05 73.025) (end 146.05 72.136) (width 0.25) (layer F.Cu) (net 12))
 (segment (start 146.812 71.374) (end 147.701 71.374) (width 0.25) (layer F.Cu) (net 12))
 (segment (start 146.05 72.136) (end 146.812 71.374) (width 0.25) (layer F.Cu) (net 12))
 (segment (start 151.765 70.231) (end 151.765 69.85) (width 0.25) (layer F.Cu) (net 13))
 (segment (start 150.622 71.374) (end 151.765 70.231) (width 0.25) (layer F.Cu) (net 13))
 (segment (start 160.02 69.342) (end 160.02 70.485) (width 0.25) (layer F.Cu) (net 13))
 (segment (start 152.146 68.58) (end 159.258 68.58) (width 0.25) (layer F.Cu) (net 13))
 (segment (start 159.258 68.58) (end 160.02 69.342) (width 0.25) (layer F.Cu) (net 13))
 (segment (start 151.765 69.85) (end 151.765 68.961) (width 0.25) (layer F.Cu) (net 13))
 (segment (start 151.765 68.961) (end 152.146 68.58) (width 0.25) (layer F.Cu) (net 13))
 (segment (start 148.59 73.025) (end 148.59 72.136) (width 0.25) (layer F.Cu) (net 13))
 (segment (start 149.352 71.374) (end 150.622 71.374) (width 0.25) (layer F.Cu) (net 13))
 (segment (start 148.59 72.136) (end 149.352 71.374) (width 0.25) (layer F.Cu) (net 13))
 (segment (start 167.132 72.898) (end 167.64 72.39) (width 0.25) (layer F.Cu) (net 14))
 (segment (start 167.64 72.39) (end 167.64 71.560001) (width 0.25) (layer F.Cu) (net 14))
 (segment (start 167.64 71.560001) (end 167.64 70.485) (width 0.25) (layer F.Cu) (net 14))
 (segment (start 155.104999 70.649999) (end 155.104999 70.776999) (width 0.25) (layer F.Cu) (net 14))
 (segment (start 154.305 69.85) (end 155.104999 70.649999) (width 0.25) (layer F.Cu) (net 14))
 (segment (start 155.104999 70.776999) (end 155.702 71.374) (width 0.25) (layer F.Cu) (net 14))
 (segment (start 155.702 71.374) (end 157.734 71.374) (width 0.25) (layer F.Cu) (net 14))
 (segment (start 159.258 72.898) (end 167.132 72.898) (width 0.25) (layer F.Cu) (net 14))
 (segment (start 157.734 71.374) (end 159.258 72.898) (width 0.25) (layer F.Cu) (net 14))
 (segment (start 151.13 73.025) (end 151.13 72.644) (width 0.25) (layer F.Cu) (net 14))
 (segment (start 151.13 72.644) (end 152.4 71.374) (width 0.25) (layer F.Cu) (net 14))
 (segment (start 153.505001 70.649999) (end 153.505001 70.776999) (width 0.25) (layer F.Cu) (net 14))
 (segment (start 154.305 69.85) (end 153.505001 70.649999) (width 0.25) (layer F.Cu) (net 14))
 (segment (start 152.908 71.374) (end 152.4 71.374) (width 0.25) (layer F.Cu) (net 14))
 (segment (start 153.505001 70.776999) (end 152.908 71.374) (width 0.25) (layer F.Cu) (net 14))
 (segment (start 154.305 77.47) (end 154.305 78.613) (width 0.25) (layer F.Cu) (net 15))
 (segment (start 154.305 78.613) (end 153.67 79.248) (width 0.25) (layer F.Cu) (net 15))
 (segment (start 153.67 79.248) (end 153.67 80.645) (width 0.25) (layer F.Cu) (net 15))
 (segment (start 155.10684 80.645) (end 156.21 80.645) (width 0.25) (layer F.Cu) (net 15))
 (segment (start 153.67 80.645) (end 155.10684 80.645) (width 0.25) (layer F.Cu) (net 15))
 (segment (start 125.594 72.254) (end 125.476 72.136) (width 0.25) (layer B.Cu) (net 5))
 (segment (start 127.889 72.254) (end 125.594 72.254) (width 0.25) (layer B.Cu) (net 5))
 (segment (start 141.605 69.85) (end 141.605 68.199) (width 0.25) (layer F.Cu) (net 5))
 (segment (start 125.476 69.596) (end 125.476 72.136) (width 0.25) (layer F.Cu) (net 5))
 (segment (start 127.254 67.818) (end 125.476 69.596) (width 0.25) (layer F.Cu) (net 5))
 (segment (start 140.97 67.818) (end 127.254 67.818) (width 0.25) (layer F.Cu) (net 5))
 (segment (start 141.605 68.199) (end 141.351 68.199) (width 0.25) (layer F.Cu) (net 5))
 (segment (start 141.351 68.199) (end 140.97 67.818) (width 0.25) (layer F.Cu) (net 5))
 (segment (start 127.855 77.47) (end 128.905 77.47) (width 0.25) (layer B.Cu) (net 1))
 (segment (start 127.508 77.817) (end 127.855 77.47) (width 0.25) (layer B.Cu) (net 1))
 (segment (start 127.508 81.364) (end 127.508 77.817) (width 0.25) (layer B.Cu) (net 1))
 (segment (start 126.576 82.296) (end 127.508 81.364) (width 0.25) (layer B.Cu) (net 1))
 (segment (start 125.476 82.296) (end 126.576 82.296) (width 0.25) (layer B.Cu) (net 1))
 (segment (start 129.286 81.026) (end 128.016 79.756) (width 0.25) (layer F.Cu) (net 2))
 (segment (start 157.644999 78.269999) (end 158.025999 78.269999) (width 0.25) (layer F.Cu) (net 2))
 (segment (start 158.242 81.788) (end 157.734 82.296) (width 0.25) (layer F.Cu) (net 2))
 (segment (start 158.025999 78.269999) (end 158.242 78.486) (width 0.25) (layer F.Cu) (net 2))
 (segment (start 128.016 79.756) (end 125.476 79.756) (width 0.25) (layer F.Cu) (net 2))
 (segment (start 156.845 77.47) (end 157.644999 78.269999) (width 0.25) (layer F.Cu) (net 2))
 (segment (start 158.242 78.486) (end 158.242 81.788) (width 0.25) (layer F.Cu) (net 2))
 (segment (start 129.286 81.026) (end 130.556 82.296) (width 0.25) (layer F.Cu) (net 2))
 (segment (start 157.734 82.296) (end 130.556 82.296) (width 0.25) (layer F.Cu) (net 2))
 (segment (start 156.845 68.961) (end 156.845 69.85) (width 0.25) (layer B.Cu) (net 3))
 (segment (start 155.956 68.072) (end 156.845 68.961) (width 0.25) (layer B.Cu) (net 3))
 (segment (start 125.476 77.216) (end 127 75.692) (width 0.25) (layer B.Cu) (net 3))
 (segment (start 127 75.692) (end 129.667 75.692) (width 0.25) (layer B.Cu) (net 3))
 (segment (start 129.667 75.692) (end 129.921 75.438) (width 0.25) (layer B.Cu) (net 3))
 (segment (start 129.921 75.438) (end 129.921 71.374) (width 0.25) (layer B.Cu) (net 3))
 (segment (start 129.921 71.374) (end 130.175 71.12) (width 0.25) (layer B.Cu) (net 3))
 (segment (start 130.175 68.707) (end 130.81 68.072) (width 0.25) (layer B.Cu) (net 3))
 (segment (start 130.175 71.12) (end 130.175 68.707) (width 0.25) (layer B.Cu) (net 3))
 (segment (start 130.81 68.072) (end 155.956 68.072) (width 0.25) (layer B.Cu) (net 3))
 (segment (start 144.145 68.689) (end 143.655 68.199) (width 0.25) (layer F.Cu) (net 17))
 (segment (start 144.145 69.85) (end 144.145 68.689) (width 0.25) (layer F.Cu) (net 17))
 (segment (start 171.831 70.485) (end 170.18 70.485) (width 0.25) (layer B.Cu) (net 18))
 (segment (start 172.212 81.915) (end 172.212 70.866) (width 0.25) (layer B.Cu) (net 18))
 (segment (start 171.577 82.55) (end 172.212 81.915) (width 0.25) (layer B.Cu) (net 18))
 (segment (start 159.258 82.55) (end 171.577 82.55) (width 0.25) (layer B.Cu) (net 18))
 (segment (start 141.605 78.60137) (end 141.99763 78.994) (width 0.25) (layer B.Cu) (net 18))
 (segment (start 172.212 70.866) (end 171.831 70.485) (width 0.25) (layer B.Cu) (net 18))
 (segment (start 141.605 77.47) (end 141.605 78.60137) (width 0.25) (layer B.Cu) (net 18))
 (segment (start 141.99763 78.994) (end 157.734 78.994) (width 0.25) (layer B.Cu) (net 18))
 (segment (start 158.242 81.534) (end 159.258 82.55) (width 0.25) (layer B.Cu) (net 18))
 (segment (start 157.734 78.994) (end 158.242 79.502) (width 0.25) (layer B.Cu) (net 18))
 (segment (start 158.242 79.502) (end 158.242 81.534) (width 0.25) (layer B.Cu) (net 18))
 (segment (start 144.145 76.33863) (end 144.526 75.95763) (width 0.25) (layer F.Cu) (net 19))
 (segment (start 144.145 77.47) (end 144.145 76.33863) (width 0.25) (layer F.Cu) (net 19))
 (segment (start 144.526 75.95763) (end 144.526 75.946) (width 0.25) (layer F.Cu) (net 19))
 (segment (start 144.526 75.946) (end 144.907 75.565) (width 0.25) (layer F.Cu) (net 19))
 (segment (start 144.907 75.565) (end 158.242 75.565) (width 0.25) (layer F.Cu) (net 19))
 (segment (start 158.242 75.565) (end 160.02 77.343) (width 0.25) (layer F.Cu) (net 19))
 (segment (start 160.02 77.343) (end 160.02 80.645) (width 0.25) (layer F.Cu) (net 19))
 (segment (start 136.525 78.60137) (end 136.525 77.47) (width 0.25) (layer F.Cu) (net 4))
 (segment (start 137.033 79.10937) (end 136.525 78.60137) (width 0.25) (layer F.Cu) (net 4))
 (segment (start 148.717 79.10937) (end 137.033 79.10937) (width 0.25) (layer F.Cu) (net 4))
 (segment (start 149.225 78.60137) (end 148.717 79.10937) (width 0.25) (layer F.Cu) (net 4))
 (segment (start 149.225 77.47) (end 149.225 78.60137) (width 0.25) (layer F.Cu) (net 4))
 (segment (start 125.848 74.304) (end 125.476 74.676) (width 0.25) (layer B.Cu) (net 4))
 (segment (start 127.889 74.304) (end 125.848 74.304) (width 0.25) (layer B.Cu) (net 4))
 (segment (start 136.144 75.692) (end 127.508 75.692) (width 0.25) (layer F.Cu) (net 4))
 (segment (start 136.525 77.47) (end 136.525 76.073) (width 0.25) (layer F.Cu) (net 4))
 (segment (start 126.492 74.676) (end 125.476 74.676) (width 0.25) (layer F.Cu) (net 4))
 (segment (start 127.508 75.692) (end 126.492 74.676) (width 0.25) (layer F.Cu) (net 4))
 (segment (start 136.525 76.073) (end 136.144 75.692) (width 0.25) (layer F.Cu) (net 4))
 (segment (start 129.782372 79.132628) (end 129.159 79.756) (width 0.25) (layer B.Cu) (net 16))
 (segment (start 130.671372 79.132628) (end 129.782372 79.132628) (width 0.25) (layer B.Cu) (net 16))
 (segment (start 131.445 77.47) (end 131.445 78.359) (width 0.25) (layer B.Cu) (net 16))
 (segment (start 131.445 78.359) (end 130.671372 79.132628) (width 0.25) (layer B.Cu) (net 16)))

